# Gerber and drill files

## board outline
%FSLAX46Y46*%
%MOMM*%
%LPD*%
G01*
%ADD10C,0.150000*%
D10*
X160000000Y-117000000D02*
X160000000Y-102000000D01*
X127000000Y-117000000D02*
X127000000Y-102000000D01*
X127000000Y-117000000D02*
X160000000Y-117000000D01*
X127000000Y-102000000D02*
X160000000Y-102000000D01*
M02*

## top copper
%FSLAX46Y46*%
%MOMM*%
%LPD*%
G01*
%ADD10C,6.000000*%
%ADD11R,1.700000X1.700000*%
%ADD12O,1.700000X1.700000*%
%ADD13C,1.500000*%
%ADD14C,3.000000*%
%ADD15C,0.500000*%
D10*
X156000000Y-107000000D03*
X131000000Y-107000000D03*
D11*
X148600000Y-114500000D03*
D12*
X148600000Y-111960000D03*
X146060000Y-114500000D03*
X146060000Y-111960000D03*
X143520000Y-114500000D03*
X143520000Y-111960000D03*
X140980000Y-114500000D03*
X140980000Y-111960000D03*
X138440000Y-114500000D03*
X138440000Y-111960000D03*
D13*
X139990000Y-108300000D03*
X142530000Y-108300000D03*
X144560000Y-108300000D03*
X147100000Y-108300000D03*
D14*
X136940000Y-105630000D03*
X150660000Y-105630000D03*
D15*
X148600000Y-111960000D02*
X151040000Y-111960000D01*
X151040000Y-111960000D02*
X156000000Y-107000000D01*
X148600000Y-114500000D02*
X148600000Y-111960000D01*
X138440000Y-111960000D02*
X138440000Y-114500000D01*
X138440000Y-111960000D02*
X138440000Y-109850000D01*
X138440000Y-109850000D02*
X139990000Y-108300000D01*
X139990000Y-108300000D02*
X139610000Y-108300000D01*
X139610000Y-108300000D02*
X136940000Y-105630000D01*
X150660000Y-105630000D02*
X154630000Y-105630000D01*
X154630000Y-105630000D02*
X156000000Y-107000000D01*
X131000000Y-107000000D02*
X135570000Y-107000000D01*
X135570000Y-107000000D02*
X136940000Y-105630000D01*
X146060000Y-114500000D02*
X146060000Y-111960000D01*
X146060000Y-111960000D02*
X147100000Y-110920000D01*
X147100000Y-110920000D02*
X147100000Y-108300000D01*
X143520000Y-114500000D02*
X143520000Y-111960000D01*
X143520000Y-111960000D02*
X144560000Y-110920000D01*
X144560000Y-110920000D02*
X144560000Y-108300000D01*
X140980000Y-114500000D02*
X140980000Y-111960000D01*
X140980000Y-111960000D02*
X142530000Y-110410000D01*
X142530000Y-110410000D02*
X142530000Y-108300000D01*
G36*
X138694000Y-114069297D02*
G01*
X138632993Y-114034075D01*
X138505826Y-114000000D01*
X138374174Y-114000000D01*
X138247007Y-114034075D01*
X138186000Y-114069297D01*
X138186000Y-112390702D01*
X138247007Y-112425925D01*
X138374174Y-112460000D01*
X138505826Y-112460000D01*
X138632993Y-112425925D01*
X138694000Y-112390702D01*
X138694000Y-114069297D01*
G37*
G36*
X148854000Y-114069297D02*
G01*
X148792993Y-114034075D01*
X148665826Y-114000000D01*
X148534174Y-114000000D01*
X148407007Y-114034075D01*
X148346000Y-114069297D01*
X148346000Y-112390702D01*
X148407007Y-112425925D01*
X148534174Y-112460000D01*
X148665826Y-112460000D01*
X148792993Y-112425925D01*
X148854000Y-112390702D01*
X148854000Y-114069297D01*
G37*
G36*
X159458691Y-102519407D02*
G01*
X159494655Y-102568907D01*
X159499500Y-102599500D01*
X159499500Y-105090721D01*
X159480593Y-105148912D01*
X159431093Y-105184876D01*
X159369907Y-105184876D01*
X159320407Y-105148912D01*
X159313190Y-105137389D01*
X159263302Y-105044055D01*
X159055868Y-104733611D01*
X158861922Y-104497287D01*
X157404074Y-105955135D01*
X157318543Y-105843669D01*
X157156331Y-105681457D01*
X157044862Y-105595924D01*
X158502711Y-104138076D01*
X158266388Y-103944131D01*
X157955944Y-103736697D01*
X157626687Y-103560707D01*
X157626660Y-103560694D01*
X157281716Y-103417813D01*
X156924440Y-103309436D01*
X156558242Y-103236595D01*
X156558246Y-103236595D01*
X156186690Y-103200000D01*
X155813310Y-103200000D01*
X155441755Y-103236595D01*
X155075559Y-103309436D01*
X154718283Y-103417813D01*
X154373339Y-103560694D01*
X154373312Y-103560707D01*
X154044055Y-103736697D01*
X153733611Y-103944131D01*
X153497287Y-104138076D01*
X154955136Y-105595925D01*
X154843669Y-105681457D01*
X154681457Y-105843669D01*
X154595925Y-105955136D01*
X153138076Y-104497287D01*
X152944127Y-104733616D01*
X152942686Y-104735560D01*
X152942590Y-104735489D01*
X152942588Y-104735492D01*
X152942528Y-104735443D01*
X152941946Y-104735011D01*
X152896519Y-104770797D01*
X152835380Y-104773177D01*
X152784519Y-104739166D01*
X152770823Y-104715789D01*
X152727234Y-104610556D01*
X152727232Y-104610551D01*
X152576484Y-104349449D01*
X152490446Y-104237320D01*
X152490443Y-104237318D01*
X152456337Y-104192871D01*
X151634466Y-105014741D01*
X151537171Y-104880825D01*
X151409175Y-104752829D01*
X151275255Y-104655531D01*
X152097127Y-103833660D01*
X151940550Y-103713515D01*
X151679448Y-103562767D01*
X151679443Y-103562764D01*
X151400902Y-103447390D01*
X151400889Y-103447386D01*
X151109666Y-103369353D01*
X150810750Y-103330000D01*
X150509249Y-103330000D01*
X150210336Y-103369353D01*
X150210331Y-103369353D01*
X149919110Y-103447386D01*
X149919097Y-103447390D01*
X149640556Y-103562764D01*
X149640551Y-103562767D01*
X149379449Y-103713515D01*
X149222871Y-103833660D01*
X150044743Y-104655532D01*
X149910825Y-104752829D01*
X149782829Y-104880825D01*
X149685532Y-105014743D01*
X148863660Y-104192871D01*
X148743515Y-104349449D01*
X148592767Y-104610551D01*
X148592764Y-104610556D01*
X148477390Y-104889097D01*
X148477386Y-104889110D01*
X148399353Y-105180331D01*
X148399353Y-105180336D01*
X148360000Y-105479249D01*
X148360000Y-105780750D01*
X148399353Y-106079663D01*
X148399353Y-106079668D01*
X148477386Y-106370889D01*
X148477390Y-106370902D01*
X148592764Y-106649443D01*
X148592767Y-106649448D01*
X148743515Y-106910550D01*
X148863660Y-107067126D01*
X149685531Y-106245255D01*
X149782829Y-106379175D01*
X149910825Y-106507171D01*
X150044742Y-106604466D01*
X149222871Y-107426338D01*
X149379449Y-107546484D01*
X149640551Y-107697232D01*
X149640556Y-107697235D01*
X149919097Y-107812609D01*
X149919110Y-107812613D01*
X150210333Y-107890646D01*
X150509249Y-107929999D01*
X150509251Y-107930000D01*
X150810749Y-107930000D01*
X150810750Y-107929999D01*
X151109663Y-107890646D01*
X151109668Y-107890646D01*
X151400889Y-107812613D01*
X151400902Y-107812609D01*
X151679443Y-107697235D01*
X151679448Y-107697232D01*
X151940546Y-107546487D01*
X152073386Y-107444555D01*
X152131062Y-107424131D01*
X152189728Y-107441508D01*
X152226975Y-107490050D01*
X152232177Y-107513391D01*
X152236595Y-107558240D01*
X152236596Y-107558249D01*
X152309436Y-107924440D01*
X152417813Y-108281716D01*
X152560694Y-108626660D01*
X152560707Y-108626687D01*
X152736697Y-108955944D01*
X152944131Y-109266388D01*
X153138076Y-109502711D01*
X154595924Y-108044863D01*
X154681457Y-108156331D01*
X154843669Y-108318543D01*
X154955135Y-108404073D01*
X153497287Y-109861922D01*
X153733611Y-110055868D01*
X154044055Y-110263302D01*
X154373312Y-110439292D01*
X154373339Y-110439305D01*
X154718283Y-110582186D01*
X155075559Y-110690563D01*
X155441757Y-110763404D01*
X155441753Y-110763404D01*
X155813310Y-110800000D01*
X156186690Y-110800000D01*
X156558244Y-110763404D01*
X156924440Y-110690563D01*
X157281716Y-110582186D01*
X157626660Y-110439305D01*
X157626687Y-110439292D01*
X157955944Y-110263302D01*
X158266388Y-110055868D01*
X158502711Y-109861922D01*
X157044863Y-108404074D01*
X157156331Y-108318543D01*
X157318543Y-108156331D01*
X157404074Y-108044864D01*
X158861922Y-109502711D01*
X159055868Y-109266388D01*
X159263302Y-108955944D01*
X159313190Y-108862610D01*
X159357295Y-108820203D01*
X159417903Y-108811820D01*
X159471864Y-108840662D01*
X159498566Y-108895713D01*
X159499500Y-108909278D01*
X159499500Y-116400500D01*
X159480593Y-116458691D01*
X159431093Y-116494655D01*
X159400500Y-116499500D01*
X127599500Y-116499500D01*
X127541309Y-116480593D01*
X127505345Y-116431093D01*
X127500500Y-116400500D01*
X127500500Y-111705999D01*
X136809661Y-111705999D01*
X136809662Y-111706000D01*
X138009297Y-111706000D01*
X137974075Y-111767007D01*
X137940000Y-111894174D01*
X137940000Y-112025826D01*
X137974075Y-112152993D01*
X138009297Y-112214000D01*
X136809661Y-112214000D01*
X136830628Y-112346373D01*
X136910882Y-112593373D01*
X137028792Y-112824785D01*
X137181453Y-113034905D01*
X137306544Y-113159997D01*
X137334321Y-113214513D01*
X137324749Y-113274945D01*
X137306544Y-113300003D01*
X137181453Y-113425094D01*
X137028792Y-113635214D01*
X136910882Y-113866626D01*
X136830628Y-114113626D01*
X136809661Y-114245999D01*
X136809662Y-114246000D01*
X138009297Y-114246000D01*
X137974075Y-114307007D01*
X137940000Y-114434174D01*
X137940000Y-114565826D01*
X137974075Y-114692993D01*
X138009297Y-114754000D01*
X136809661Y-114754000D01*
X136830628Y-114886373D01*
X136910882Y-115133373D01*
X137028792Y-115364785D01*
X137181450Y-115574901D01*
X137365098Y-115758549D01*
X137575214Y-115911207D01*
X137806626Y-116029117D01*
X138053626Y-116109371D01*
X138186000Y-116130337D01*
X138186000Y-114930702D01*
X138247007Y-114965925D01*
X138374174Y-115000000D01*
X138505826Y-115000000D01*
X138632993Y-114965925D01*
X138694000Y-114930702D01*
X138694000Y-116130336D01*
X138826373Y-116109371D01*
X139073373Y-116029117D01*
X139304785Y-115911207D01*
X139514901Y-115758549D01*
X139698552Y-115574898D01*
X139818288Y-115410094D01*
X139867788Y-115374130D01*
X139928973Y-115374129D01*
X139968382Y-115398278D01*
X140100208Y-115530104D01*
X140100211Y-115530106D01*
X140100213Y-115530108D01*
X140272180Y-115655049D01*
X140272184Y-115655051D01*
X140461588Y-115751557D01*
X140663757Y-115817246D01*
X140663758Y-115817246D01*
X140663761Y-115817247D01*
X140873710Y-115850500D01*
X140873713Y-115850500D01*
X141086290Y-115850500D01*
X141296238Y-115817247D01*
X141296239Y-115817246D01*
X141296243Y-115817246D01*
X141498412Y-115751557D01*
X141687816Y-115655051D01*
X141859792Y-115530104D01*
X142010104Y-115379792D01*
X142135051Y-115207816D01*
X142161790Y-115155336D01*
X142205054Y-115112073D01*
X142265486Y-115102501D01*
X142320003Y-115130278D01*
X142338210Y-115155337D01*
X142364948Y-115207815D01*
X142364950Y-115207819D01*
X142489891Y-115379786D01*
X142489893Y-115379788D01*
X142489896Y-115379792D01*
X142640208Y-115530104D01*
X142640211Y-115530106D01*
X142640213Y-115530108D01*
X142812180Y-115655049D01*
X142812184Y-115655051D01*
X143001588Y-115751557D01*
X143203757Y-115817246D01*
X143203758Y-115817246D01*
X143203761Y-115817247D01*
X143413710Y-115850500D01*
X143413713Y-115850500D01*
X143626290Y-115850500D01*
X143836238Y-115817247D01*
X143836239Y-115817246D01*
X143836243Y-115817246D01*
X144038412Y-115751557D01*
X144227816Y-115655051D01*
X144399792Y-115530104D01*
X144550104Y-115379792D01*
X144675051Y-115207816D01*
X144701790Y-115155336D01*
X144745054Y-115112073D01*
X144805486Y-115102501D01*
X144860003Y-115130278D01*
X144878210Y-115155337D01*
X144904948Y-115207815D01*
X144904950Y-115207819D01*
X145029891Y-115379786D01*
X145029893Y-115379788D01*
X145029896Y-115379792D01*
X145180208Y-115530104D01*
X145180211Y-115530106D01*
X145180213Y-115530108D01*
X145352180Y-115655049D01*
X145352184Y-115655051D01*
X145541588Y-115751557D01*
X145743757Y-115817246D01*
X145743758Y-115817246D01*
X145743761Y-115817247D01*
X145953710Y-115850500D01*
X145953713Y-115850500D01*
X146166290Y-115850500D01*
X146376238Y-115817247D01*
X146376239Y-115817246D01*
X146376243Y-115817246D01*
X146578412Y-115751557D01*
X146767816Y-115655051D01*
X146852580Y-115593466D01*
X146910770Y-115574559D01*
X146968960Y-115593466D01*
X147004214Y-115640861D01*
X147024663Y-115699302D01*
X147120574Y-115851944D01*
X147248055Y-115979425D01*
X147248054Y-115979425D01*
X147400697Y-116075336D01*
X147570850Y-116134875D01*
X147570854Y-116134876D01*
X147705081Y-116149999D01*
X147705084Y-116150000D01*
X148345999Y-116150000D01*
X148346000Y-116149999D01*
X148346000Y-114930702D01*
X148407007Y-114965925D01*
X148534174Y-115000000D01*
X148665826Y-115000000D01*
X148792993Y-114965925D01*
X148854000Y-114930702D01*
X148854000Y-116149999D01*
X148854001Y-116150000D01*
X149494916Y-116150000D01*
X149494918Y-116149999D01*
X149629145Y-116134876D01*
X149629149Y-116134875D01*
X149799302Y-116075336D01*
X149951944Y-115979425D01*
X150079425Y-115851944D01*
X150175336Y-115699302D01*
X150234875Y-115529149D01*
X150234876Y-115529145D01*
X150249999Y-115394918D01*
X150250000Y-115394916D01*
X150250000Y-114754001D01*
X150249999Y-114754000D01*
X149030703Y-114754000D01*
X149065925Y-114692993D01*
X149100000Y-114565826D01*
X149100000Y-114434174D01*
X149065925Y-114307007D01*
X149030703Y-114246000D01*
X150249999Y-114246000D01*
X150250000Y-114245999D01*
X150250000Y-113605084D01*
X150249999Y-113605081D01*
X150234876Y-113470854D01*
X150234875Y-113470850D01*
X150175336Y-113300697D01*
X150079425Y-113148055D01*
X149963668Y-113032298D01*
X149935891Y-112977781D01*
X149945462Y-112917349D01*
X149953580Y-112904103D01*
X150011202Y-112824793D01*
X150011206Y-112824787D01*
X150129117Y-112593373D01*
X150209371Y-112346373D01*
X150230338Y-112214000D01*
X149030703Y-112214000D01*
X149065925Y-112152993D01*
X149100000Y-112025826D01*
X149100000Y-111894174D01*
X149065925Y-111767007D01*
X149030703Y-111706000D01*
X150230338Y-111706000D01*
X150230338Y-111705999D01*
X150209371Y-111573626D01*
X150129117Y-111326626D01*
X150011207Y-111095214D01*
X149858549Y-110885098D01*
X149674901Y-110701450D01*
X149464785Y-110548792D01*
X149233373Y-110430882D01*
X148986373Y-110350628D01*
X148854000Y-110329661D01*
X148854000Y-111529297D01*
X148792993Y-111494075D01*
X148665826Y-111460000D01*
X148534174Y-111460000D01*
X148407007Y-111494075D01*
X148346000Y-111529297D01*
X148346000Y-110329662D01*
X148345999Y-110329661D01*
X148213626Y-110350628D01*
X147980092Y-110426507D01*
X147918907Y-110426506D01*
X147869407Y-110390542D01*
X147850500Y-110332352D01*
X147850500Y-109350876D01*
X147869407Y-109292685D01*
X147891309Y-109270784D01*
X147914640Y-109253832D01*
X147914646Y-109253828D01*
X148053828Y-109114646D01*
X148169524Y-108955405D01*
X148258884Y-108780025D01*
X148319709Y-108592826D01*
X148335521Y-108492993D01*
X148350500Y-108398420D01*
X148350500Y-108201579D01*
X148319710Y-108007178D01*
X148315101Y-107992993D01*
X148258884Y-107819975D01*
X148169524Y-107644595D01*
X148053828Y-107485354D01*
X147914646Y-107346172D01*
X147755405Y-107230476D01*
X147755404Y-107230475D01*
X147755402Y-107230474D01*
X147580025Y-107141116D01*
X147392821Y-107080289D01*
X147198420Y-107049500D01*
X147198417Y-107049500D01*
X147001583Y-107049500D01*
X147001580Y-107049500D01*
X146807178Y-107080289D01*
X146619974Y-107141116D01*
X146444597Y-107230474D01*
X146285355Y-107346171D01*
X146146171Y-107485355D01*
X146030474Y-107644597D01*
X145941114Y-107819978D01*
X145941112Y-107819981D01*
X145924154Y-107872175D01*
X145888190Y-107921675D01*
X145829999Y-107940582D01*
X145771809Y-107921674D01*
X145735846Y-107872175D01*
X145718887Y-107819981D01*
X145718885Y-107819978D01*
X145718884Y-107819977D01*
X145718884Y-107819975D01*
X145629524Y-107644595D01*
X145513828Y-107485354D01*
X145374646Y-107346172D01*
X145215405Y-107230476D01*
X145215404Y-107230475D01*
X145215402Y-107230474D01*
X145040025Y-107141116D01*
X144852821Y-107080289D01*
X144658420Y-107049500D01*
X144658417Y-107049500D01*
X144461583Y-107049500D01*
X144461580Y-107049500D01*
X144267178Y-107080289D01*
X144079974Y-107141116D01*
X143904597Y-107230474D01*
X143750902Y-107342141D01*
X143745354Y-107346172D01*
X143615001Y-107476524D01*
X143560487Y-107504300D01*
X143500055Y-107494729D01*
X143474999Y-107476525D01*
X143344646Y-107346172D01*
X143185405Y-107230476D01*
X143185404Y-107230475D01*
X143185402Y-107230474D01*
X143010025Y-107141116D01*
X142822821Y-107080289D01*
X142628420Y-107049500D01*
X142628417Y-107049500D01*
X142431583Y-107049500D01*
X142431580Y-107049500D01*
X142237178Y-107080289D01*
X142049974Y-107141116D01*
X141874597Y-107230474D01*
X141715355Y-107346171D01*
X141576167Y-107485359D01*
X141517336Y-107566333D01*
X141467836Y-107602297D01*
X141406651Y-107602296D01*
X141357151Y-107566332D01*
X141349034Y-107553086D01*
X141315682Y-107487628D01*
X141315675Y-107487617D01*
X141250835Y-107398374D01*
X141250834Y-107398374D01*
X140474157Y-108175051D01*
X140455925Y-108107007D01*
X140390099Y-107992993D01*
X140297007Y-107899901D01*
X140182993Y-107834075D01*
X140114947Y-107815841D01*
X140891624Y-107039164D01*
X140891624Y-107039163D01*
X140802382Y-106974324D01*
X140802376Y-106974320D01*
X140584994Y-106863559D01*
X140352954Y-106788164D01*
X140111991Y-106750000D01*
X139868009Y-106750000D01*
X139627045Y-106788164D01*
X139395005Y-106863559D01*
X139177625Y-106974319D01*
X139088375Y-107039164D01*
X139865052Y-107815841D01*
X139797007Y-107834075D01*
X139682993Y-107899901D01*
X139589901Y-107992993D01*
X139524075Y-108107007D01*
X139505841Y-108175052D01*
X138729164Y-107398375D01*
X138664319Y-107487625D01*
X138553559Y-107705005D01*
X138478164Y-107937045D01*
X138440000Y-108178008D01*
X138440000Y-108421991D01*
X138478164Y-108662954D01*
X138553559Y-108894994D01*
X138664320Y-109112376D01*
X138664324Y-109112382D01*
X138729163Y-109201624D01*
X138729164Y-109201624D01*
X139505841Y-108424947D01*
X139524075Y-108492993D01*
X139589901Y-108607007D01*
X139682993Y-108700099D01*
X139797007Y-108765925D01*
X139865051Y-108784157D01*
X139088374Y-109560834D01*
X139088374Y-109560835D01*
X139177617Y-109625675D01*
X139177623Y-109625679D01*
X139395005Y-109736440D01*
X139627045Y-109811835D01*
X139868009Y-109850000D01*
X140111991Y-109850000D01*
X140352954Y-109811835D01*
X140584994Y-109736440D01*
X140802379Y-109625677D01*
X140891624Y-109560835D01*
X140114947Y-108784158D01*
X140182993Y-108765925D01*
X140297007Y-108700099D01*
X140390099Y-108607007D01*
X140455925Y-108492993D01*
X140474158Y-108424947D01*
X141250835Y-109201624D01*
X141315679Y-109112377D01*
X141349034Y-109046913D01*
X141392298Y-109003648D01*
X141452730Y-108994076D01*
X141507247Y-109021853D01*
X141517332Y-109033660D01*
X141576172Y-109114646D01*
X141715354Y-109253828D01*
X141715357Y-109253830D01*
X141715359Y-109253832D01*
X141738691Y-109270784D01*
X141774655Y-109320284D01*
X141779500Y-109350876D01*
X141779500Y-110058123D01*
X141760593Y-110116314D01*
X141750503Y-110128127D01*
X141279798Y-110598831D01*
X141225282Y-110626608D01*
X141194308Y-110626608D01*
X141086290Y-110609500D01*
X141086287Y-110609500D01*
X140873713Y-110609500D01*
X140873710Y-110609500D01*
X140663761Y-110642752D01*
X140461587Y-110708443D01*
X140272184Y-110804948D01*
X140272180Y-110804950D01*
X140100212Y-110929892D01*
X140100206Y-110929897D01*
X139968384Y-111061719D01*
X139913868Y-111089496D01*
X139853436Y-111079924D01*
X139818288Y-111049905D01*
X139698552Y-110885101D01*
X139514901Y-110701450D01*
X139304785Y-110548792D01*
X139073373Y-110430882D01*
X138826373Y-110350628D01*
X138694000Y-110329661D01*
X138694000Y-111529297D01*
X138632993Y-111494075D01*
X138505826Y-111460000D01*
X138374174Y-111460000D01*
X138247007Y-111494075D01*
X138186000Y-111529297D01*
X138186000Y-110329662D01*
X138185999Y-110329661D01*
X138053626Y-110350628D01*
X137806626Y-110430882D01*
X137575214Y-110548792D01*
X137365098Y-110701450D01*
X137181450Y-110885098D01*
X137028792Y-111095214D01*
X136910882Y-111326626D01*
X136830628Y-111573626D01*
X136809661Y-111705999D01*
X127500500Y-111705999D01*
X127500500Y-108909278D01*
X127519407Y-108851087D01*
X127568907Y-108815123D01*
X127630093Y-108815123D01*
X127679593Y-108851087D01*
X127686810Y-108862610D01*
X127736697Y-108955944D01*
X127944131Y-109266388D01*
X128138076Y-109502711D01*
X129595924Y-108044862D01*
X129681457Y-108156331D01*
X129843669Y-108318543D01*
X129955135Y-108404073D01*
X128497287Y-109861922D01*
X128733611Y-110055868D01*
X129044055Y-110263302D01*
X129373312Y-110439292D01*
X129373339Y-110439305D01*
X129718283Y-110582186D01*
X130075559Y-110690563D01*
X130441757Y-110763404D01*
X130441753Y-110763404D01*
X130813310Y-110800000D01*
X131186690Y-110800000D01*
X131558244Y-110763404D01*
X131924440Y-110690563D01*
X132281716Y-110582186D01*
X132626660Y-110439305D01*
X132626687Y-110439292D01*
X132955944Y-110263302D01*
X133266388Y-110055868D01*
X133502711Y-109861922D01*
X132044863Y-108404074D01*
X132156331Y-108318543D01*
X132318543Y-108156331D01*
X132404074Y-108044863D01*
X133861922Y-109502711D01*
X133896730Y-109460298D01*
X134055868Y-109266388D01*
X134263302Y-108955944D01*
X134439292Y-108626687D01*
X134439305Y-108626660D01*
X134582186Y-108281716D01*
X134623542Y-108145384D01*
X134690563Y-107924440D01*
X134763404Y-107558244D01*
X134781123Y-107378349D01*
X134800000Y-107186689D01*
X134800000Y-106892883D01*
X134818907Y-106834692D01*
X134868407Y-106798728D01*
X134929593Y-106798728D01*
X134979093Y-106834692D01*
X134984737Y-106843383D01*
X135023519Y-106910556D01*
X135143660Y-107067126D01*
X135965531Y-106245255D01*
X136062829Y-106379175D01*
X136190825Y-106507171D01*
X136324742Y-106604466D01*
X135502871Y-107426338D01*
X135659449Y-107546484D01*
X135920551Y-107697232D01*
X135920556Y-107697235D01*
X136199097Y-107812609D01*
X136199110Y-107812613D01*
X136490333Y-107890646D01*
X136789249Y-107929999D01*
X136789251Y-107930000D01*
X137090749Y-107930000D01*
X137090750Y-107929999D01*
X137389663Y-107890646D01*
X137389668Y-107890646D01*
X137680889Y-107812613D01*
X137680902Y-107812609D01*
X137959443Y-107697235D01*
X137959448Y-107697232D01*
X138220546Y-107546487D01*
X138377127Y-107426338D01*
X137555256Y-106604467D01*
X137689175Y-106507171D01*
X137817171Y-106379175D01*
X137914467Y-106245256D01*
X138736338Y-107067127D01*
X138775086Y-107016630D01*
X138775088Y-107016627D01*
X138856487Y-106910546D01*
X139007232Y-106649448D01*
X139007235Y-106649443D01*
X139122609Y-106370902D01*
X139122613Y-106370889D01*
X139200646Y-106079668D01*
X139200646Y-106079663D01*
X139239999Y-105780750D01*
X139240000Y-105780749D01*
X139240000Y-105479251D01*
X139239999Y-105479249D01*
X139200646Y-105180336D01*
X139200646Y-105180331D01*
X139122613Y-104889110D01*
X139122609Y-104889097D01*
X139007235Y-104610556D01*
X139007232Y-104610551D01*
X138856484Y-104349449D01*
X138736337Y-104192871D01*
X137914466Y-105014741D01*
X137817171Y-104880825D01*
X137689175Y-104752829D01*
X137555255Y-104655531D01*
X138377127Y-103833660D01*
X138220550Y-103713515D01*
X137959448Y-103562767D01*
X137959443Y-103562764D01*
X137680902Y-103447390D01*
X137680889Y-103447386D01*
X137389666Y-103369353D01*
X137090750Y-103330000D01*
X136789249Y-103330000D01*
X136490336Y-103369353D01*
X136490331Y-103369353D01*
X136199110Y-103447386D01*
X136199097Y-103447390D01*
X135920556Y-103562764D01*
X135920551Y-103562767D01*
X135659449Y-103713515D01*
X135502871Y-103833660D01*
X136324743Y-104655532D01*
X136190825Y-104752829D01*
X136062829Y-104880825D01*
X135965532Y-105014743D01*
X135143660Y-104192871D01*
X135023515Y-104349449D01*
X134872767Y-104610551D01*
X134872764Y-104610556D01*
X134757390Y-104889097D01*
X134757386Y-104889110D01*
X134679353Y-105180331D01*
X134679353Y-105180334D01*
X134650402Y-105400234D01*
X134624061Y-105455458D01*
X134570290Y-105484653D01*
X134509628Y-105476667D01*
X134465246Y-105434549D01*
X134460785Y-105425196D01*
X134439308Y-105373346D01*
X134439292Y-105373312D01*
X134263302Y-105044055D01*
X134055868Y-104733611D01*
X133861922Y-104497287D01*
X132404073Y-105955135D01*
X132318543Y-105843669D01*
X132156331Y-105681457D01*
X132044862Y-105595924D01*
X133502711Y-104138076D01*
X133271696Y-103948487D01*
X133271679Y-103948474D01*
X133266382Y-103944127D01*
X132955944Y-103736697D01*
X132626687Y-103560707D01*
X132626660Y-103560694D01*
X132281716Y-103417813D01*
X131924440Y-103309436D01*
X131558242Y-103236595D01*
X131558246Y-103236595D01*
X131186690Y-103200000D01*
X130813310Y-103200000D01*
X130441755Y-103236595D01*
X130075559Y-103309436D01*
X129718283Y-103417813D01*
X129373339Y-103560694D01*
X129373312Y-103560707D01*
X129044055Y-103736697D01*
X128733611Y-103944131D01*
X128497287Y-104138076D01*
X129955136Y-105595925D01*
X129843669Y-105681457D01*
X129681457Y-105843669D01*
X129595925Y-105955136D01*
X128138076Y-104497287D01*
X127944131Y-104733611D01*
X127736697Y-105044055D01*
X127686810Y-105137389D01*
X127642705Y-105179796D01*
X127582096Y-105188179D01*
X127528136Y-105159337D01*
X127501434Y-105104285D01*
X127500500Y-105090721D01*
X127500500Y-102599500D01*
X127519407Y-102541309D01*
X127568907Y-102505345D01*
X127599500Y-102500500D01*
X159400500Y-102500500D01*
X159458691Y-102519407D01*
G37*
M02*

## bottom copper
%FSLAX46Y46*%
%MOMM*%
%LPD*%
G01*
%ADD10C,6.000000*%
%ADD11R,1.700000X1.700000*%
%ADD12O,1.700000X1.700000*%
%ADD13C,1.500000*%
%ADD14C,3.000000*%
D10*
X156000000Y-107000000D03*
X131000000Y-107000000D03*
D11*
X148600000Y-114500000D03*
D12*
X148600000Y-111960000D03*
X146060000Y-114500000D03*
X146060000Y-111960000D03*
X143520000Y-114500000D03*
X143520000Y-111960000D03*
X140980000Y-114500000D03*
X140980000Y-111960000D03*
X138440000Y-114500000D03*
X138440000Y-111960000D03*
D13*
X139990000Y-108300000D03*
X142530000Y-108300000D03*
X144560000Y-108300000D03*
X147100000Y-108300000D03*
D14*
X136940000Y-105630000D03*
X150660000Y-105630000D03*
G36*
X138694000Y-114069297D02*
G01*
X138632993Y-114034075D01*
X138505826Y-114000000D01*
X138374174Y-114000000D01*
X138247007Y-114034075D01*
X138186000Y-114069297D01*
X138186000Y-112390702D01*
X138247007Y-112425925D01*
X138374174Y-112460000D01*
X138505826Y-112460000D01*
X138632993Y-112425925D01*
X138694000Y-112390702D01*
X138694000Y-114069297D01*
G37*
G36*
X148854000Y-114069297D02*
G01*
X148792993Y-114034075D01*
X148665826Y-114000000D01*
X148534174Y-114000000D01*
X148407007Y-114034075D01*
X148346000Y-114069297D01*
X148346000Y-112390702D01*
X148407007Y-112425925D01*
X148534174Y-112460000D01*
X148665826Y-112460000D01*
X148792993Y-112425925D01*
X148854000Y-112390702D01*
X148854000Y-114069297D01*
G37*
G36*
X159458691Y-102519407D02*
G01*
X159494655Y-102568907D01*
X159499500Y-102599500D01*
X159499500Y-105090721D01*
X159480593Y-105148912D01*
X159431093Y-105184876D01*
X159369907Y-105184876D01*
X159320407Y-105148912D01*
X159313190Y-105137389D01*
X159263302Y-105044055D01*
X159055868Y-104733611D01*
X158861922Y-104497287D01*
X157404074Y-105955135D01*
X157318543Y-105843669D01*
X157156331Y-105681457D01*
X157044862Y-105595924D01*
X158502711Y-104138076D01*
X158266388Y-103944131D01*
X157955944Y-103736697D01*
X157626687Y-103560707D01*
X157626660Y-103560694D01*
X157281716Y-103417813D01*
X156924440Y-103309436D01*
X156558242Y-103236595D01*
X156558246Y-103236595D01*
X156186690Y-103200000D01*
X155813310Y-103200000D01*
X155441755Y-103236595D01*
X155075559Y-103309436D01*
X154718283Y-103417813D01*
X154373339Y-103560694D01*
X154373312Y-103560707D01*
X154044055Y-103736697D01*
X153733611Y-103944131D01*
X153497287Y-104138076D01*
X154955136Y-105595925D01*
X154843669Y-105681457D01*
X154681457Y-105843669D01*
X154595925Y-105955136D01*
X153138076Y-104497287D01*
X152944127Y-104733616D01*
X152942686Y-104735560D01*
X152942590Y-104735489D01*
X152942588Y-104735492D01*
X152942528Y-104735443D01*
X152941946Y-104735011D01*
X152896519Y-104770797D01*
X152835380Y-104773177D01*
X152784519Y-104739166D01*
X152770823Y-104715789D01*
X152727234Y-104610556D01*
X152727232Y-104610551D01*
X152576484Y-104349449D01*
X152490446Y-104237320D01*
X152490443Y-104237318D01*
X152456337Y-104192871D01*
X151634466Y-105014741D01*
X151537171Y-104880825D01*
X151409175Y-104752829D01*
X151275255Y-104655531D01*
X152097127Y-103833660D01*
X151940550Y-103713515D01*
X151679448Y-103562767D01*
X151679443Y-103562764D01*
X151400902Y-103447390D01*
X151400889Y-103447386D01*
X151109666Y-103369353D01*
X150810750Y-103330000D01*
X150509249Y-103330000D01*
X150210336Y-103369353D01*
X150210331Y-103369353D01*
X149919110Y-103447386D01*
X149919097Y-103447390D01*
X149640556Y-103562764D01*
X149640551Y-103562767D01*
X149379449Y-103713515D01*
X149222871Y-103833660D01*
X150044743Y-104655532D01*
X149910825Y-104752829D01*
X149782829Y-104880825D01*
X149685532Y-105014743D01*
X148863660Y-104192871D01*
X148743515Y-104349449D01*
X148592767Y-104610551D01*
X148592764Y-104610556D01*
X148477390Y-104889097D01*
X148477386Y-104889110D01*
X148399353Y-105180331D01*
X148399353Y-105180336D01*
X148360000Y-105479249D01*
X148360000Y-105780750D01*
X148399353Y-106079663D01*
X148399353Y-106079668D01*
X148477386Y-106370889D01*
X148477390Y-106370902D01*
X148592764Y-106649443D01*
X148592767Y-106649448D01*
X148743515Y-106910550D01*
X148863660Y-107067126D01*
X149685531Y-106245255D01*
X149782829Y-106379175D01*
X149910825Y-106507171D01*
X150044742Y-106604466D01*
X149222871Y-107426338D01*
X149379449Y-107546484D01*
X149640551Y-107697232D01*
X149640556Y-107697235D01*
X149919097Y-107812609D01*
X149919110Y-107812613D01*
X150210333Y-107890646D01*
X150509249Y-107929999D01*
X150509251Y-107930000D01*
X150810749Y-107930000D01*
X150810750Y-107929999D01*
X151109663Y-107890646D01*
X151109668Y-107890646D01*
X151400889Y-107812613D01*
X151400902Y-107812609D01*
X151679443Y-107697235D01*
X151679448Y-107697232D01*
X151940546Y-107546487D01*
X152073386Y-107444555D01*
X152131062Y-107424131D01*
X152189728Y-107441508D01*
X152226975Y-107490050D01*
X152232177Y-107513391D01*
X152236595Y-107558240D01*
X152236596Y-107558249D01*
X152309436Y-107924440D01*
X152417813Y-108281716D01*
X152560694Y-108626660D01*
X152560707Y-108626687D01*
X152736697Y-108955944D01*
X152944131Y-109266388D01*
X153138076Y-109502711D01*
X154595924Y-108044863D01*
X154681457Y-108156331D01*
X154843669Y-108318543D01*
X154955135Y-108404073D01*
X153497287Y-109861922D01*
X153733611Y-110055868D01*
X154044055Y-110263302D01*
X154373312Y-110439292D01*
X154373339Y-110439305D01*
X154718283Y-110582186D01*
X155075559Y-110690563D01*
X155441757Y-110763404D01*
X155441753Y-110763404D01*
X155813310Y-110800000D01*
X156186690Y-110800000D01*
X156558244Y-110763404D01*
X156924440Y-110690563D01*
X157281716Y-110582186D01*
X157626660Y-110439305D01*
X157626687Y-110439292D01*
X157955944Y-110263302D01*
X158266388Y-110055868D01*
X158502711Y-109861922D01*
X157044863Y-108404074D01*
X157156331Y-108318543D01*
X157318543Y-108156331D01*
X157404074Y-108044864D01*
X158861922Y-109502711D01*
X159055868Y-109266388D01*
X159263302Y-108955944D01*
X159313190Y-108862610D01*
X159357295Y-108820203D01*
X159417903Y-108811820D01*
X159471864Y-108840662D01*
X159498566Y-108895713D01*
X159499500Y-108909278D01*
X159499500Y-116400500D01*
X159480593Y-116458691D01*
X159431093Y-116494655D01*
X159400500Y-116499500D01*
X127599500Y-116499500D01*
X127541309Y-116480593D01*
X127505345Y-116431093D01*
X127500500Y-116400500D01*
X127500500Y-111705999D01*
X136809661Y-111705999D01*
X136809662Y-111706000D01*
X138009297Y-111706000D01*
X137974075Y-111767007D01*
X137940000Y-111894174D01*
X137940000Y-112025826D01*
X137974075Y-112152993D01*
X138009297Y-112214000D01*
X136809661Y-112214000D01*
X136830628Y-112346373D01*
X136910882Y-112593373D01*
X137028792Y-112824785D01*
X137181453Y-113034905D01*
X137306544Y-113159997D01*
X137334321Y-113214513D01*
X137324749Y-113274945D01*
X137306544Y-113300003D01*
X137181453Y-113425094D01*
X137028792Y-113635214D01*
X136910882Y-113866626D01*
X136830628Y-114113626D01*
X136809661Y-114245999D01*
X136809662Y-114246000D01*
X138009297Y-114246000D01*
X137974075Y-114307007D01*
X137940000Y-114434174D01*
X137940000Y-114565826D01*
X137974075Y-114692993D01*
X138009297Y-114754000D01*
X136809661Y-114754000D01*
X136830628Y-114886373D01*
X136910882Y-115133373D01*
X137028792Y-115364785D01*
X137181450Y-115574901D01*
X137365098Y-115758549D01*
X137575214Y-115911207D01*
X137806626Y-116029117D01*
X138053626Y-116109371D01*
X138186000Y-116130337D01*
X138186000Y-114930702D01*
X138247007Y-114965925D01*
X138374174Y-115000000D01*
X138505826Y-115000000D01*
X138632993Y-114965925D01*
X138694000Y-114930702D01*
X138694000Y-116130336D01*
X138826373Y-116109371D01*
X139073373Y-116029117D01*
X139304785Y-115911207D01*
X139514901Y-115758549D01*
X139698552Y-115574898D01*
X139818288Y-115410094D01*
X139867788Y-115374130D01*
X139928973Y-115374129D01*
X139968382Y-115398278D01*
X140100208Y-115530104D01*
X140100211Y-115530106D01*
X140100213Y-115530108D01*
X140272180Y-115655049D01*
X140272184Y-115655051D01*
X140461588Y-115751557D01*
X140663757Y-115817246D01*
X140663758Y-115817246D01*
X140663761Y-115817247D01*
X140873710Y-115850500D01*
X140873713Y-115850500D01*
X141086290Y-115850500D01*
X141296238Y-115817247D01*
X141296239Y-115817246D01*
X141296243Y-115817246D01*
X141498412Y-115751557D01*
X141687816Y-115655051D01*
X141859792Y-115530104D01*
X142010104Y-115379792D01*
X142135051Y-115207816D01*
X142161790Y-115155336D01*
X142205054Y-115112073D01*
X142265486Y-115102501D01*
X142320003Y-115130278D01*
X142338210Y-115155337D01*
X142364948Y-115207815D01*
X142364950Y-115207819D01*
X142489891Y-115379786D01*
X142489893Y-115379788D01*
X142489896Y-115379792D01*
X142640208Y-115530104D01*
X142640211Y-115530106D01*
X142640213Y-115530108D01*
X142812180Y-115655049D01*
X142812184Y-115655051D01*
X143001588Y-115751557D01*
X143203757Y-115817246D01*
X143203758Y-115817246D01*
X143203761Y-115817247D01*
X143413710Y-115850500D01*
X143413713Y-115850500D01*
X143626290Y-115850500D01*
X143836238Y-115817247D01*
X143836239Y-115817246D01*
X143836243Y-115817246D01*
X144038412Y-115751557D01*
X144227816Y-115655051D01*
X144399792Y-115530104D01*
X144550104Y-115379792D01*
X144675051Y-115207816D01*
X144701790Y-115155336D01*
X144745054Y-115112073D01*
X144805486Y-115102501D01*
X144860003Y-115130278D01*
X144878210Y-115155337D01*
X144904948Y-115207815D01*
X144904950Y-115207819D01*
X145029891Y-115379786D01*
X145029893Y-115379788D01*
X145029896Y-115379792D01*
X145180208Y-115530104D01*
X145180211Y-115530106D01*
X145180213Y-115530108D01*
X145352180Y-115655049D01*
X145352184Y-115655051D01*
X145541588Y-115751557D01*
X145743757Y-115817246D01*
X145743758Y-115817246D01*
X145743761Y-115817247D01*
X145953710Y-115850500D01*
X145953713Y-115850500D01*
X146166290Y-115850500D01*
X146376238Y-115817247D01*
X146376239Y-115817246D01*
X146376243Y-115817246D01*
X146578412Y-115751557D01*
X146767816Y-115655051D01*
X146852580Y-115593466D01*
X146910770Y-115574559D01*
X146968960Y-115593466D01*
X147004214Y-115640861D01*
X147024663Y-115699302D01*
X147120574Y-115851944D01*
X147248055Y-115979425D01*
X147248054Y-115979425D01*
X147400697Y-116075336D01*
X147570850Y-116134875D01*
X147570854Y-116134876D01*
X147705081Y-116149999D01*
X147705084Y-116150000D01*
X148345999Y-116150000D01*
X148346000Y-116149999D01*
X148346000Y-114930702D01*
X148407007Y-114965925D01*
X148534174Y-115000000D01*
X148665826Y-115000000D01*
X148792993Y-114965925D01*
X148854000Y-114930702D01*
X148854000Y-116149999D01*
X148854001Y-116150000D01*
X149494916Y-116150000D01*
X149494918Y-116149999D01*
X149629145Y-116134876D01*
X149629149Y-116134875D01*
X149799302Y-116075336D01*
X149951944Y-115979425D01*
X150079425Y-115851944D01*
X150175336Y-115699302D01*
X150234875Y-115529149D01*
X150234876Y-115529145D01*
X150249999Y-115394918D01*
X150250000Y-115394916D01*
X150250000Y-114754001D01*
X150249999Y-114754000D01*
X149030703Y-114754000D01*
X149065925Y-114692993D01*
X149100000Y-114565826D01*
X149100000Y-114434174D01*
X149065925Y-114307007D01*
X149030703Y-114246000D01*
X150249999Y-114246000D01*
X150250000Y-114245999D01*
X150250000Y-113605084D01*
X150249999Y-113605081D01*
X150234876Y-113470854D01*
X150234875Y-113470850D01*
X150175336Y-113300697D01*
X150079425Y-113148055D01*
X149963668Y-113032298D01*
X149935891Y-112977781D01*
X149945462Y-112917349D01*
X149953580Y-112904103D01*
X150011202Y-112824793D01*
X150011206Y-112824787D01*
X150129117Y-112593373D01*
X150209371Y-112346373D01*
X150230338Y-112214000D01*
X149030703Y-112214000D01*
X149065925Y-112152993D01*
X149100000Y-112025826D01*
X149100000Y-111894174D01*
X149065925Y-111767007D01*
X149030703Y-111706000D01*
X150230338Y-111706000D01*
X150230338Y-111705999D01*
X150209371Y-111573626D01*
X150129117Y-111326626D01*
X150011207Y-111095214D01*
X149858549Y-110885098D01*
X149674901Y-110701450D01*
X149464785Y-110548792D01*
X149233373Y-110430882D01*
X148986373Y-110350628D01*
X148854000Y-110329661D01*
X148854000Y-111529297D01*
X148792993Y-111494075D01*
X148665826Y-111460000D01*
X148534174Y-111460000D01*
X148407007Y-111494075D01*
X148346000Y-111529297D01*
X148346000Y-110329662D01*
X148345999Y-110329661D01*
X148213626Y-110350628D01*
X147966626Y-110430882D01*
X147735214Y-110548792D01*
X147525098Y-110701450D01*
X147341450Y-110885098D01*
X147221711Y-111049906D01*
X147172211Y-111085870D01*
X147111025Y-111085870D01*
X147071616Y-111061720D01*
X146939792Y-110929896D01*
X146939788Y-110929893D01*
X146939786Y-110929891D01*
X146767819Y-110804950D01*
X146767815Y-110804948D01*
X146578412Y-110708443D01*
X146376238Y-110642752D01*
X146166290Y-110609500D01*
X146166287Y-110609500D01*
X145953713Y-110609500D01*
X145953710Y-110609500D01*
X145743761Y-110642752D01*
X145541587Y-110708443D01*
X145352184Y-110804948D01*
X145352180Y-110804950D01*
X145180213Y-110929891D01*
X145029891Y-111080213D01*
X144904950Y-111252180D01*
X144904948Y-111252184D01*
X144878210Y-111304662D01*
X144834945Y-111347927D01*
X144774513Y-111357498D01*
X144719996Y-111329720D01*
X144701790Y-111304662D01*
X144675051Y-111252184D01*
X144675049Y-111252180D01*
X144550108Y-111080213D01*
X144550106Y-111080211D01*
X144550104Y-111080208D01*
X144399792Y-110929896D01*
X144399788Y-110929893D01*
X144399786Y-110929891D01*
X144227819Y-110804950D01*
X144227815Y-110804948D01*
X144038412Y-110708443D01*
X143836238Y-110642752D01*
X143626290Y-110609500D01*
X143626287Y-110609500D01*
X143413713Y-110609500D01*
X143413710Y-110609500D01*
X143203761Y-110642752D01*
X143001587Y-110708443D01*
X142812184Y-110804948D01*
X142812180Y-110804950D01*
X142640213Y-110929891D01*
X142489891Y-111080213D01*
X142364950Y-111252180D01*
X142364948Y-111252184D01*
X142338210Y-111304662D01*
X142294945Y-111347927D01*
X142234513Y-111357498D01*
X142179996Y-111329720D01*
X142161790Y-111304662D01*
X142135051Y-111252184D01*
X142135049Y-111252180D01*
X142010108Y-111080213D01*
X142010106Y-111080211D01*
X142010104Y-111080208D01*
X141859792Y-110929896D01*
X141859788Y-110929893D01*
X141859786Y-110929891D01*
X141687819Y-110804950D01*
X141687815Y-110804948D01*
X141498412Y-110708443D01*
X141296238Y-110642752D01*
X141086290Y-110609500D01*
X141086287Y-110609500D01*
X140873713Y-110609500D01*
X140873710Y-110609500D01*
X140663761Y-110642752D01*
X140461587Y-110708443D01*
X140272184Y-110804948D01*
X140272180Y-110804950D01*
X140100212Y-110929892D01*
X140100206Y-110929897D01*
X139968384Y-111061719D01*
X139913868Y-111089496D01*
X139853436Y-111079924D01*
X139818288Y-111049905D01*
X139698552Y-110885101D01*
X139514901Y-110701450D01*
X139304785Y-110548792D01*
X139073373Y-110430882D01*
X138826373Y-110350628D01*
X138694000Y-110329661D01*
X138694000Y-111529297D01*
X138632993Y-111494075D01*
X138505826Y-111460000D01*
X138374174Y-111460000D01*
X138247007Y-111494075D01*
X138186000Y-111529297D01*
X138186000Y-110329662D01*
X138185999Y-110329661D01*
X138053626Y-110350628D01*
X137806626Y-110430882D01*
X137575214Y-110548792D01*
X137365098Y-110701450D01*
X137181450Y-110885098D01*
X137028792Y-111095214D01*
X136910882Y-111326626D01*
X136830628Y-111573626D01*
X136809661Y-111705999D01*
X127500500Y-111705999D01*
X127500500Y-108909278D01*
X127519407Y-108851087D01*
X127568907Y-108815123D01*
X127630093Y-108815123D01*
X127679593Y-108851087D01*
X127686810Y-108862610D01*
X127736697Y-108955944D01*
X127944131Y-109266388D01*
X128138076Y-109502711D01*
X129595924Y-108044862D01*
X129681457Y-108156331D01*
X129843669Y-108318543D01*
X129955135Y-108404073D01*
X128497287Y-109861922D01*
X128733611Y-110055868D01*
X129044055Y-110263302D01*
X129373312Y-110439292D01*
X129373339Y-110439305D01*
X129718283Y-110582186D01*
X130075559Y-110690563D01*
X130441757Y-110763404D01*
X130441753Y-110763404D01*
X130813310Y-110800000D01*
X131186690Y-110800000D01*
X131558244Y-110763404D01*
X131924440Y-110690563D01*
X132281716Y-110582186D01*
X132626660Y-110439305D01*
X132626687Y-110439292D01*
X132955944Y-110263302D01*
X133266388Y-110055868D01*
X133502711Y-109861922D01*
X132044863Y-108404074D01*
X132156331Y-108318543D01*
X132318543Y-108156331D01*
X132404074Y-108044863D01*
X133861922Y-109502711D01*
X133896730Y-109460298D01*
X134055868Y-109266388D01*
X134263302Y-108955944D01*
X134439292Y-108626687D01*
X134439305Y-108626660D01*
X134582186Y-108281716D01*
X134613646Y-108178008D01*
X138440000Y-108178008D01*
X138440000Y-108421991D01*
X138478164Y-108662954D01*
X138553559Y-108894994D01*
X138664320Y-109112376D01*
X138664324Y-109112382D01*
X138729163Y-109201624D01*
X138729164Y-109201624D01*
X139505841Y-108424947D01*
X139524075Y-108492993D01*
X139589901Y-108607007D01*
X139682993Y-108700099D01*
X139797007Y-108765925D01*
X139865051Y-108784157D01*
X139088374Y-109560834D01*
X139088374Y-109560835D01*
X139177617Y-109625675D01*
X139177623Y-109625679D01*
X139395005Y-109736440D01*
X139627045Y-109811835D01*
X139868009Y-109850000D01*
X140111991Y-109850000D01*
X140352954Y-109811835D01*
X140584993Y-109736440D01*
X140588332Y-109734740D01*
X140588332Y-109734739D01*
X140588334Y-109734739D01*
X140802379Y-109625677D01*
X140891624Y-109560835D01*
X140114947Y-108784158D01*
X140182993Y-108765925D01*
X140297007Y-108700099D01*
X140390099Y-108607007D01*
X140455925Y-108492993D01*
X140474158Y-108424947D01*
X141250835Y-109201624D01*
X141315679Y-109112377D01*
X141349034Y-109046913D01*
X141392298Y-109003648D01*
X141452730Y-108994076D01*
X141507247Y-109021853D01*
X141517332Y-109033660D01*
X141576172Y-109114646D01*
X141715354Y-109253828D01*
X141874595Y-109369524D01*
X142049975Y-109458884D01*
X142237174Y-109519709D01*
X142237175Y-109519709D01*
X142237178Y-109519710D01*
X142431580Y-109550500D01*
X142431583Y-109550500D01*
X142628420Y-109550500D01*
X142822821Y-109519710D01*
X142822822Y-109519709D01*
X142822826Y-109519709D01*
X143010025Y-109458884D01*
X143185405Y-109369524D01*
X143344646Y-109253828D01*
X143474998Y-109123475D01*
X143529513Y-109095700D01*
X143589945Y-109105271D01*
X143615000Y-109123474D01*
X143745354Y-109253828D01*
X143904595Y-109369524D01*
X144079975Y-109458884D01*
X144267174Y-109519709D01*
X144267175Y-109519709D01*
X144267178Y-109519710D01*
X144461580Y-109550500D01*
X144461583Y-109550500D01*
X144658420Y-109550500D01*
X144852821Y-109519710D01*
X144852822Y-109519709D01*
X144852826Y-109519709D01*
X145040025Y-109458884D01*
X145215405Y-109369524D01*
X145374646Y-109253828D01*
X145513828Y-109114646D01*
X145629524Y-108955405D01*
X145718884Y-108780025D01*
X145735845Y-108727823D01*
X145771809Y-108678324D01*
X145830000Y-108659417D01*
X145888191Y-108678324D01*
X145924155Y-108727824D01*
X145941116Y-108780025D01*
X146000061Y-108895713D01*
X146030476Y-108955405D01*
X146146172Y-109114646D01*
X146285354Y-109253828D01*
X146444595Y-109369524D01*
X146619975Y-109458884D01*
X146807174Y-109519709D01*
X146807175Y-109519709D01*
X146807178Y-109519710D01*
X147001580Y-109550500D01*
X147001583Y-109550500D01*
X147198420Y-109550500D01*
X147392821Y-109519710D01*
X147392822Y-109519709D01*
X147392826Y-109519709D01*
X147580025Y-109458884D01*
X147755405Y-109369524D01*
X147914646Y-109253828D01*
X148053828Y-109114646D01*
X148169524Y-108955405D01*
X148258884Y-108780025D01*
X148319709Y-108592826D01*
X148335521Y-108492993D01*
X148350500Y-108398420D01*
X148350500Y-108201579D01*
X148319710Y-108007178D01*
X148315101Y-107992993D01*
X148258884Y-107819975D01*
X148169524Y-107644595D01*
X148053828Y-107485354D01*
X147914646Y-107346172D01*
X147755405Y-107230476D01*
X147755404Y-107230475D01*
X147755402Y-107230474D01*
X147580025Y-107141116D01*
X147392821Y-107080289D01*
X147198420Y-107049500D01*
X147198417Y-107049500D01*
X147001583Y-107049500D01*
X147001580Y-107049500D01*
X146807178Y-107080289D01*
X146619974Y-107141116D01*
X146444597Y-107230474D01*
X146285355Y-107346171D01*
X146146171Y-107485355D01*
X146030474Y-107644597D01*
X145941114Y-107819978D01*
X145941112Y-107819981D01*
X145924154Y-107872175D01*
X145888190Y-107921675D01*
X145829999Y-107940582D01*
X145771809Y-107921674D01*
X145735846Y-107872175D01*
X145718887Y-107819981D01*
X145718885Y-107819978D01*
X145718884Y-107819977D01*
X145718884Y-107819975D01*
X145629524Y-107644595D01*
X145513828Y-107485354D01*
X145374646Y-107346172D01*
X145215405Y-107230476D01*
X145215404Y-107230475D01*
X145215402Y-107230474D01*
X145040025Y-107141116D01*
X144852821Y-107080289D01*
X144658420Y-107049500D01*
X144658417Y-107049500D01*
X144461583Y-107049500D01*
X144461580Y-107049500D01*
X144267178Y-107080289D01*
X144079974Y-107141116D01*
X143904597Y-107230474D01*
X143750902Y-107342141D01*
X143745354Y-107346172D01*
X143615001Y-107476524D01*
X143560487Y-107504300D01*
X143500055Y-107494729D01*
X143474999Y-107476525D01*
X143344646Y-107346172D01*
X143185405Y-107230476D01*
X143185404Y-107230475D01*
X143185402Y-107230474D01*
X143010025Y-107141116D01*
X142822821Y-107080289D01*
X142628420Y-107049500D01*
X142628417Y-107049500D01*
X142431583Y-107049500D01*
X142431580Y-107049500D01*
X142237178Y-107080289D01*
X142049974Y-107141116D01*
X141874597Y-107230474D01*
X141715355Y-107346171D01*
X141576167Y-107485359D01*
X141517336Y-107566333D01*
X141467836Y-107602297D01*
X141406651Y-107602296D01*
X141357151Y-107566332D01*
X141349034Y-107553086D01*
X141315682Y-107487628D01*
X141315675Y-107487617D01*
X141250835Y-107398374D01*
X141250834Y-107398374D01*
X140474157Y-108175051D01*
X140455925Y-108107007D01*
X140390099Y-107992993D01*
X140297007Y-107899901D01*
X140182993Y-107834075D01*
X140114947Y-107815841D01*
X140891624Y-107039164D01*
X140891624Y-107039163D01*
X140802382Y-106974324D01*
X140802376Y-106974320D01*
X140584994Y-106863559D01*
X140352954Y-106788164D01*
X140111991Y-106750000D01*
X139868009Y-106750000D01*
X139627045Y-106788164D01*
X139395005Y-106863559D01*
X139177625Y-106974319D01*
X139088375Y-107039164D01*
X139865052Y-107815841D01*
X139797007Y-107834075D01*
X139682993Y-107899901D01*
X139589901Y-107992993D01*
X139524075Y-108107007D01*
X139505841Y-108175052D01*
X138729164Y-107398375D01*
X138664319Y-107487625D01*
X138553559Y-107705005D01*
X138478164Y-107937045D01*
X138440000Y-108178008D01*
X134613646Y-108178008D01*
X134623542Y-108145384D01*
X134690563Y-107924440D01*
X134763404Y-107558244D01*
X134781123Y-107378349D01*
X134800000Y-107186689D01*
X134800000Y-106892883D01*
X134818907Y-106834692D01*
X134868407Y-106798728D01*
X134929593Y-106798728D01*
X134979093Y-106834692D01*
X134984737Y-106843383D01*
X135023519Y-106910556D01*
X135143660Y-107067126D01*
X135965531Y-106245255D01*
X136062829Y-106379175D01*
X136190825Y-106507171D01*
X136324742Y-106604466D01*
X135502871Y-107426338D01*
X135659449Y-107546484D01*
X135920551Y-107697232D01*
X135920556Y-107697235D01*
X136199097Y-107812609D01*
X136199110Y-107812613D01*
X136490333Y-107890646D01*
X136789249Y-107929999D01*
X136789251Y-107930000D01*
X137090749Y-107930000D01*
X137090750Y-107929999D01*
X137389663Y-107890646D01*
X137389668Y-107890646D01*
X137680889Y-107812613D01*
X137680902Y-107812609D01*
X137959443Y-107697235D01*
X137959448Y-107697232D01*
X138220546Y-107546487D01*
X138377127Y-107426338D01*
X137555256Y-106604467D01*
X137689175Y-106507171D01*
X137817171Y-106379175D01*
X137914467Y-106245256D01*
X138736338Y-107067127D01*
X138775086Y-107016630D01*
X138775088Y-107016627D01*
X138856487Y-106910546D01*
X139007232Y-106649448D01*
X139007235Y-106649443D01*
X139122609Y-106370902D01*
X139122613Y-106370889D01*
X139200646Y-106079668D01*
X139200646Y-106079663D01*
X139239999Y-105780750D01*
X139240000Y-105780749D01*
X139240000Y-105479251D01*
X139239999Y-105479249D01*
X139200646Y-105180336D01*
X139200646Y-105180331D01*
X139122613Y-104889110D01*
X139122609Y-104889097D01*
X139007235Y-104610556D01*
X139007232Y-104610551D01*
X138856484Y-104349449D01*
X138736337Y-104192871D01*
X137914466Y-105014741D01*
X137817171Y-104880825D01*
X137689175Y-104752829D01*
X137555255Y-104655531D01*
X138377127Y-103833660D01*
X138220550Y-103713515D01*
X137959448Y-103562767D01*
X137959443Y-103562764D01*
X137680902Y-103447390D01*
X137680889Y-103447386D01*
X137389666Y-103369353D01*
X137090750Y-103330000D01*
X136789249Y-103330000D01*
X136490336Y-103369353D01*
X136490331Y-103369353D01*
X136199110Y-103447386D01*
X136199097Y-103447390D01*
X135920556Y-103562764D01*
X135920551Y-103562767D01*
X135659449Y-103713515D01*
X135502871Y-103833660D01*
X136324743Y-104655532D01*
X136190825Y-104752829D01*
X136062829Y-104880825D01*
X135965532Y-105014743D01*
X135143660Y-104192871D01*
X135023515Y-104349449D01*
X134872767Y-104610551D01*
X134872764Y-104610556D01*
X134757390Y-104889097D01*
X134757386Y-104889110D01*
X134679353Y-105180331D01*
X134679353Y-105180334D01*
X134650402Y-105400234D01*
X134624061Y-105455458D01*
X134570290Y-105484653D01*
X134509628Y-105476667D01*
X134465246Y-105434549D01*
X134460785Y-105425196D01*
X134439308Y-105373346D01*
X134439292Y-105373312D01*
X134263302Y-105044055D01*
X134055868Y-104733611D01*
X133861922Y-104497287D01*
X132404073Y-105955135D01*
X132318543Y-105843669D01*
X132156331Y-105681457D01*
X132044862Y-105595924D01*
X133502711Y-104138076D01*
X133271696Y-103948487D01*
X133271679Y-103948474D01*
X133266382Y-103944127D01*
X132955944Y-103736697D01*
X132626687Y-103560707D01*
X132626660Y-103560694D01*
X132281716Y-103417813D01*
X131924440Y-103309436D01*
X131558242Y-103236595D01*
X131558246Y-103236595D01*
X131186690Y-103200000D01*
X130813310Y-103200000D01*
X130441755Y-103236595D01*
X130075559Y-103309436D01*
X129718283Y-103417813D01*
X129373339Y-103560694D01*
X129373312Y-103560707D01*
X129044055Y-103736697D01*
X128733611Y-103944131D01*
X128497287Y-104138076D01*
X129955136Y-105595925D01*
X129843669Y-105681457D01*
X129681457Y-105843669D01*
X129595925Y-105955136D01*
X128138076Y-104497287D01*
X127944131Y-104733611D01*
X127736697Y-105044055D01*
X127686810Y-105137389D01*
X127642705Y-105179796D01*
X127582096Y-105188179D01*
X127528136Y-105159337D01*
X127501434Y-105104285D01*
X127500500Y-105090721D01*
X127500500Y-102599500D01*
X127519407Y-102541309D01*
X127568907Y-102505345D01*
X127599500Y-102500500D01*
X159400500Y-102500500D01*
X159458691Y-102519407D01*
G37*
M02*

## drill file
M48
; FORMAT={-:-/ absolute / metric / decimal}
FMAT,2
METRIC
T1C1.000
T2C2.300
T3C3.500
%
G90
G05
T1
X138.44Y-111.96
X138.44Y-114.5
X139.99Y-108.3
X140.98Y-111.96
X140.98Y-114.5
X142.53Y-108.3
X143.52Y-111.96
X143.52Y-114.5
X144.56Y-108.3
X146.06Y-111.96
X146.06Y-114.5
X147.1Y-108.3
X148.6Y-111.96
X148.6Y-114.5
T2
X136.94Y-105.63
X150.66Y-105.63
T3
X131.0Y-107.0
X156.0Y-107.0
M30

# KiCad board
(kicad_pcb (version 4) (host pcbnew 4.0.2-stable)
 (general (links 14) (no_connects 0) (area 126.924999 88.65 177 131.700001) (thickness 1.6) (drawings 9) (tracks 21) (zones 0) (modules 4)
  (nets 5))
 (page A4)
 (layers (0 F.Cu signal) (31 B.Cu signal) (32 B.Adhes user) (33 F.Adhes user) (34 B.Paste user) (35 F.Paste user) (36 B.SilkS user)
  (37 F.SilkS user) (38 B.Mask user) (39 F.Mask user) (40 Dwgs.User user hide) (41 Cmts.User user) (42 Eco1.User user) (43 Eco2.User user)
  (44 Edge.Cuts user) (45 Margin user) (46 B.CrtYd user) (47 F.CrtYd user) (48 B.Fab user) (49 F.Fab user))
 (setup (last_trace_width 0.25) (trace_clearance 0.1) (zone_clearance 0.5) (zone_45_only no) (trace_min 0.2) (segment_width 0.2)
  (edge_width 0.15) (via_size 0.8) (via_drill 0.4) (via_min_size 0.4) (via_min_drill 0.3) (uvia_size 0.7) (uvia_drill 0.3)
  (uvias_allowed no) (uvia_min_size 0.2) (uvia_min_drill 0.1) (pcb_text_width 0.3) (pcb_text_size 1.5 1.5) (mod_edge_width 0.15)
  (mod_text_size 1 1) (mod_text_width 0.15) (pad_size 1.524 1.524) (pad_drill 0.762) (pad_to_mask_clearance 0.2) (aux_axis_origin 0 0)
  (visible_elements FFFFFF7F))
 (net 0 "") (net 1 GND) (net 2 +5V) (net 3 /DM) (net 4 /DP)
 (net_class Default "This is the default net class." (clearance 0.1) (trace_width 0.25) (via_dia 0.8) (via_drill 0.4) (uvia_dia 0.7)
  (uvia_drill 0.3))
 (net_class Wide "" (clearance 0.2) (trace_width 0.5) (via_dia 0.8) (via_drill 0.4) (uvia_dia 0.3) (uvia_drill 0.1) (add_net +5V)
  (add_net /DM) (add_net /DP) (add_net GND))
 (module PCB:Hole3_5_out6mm (layer F.Cu) (at 156 107)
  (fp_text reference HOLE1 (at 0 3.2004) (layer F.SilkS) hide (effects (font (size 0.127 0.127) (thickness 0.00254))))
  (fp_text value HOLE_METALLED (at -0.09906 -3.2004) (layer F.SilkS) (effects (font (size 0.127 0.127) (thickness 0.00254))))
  (pad H thru_hole circle (at 0 0) (size 6 6) (drill 3.5) (layers *.Cu *.Mask F.SilkS) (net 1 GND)))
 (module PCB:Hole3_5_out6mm (layer F.Cu) (at 131 107)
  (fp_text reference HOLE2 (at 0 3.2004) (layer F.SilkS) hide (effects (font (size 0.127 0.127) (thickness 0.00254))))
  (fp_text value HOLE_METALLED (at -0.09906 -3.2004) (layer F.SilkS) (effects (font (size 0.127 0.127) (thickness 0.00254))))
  (pad H thru_hole circle (at 0 0) (size 6 6) (drill 3.5) (layers *.Cu *.Mask F.SilkS) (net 1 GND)))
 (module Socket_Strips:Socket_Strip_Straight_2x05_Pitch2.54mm (layer F.Cu) (at 148.6 114.5 270)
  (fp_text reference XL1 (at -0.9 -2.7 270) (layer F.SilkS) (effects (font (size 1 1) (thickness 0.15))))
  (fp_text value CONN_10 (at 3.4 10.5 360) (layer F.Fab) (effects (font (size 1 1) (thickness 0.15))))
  (pad 1 thru_hole rect (at 0 0 270) (size 1.7 1.7) (drill 1) (layers *.Cu *.Mask) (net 1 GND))
  (pad 2 thru_hole oval (at -2.54 0 270) (size 1.7 1.7) (drill 1) (layers *.Cu *.Mask) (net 1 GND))
  (pad 3 thru_hole oval (at 0 2.54 270) (size 1.7 1.7) (drill 1) (layers *.Cu *.Mask) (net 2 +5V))
  (pad 4 thru_hole oval (at -2.54 2.54 270) (size 1.7 1.7) (drill 1) (layers *.Cu *.Mask) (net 2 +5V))
  (pad 5 thru_hole oval (at 0 5.08 270) (size 1.7 1.7) (drill 1) (layers *.Cu *.Mask) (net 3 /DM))
  (pad 6 thru_hole oval (at -2.54 5.08 270) (size 1.7 1.7) (drill 1) (layers *.Cu *.Mask) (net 3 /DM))
  (pad 7 thru_hole oval (at 0 7.62 270) (size 1.7 1.7) (drill 1) (layers *.Cu *.Mask) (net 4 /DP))
  (pad 8 thru_hole oval (at -2.54 7.62 270) (size 1.7 1.7) (drill 1) (layers *.Cu *.Mask) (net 4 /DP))
  (pad 9 thru_hole oval (at 0 10.16 270) (size 1.7 1.7) (drill 1) (layers *.Cu *.Mask) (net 1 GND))
  (pad 10 thru_hole oval (at -2.54 10.16 270) (size 1.7 1.7) (drill 1) (layers *.Cu *.Mask) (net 1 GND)))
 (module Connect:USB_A (layer F.Cu) (at 147.1 108.3 180)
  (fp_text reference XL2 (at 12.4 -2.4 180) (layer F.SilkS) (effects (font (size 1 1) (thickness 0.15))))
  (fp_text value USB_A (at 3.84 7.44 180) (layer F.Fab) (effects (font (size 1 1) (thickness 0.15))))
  (pad 4 thru_hole circle (at 7.11 0 90) (size 1.5 1.5) (drill 1) (layers *.Cu *.Mask) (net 1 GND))
  (pad 3 thru_hole circle (at 4.57 0 90) (size 1.5 1.5) (drill 1) (layers *.Cu *.Mask) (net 4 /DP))
  (pad 2 thru_hole circle (at 2.54 0 90) (size 1.5 1.5) (drill 1) (layers *.Cu *.Mask) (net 3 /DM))
  (pad 1 thru_hole circle (at 0 0 90) (size 1.5 1.5) (drill 1) (layers *.Cu *.Mask) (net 2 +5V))
  (pad 5 thru_hole circle (at 10.16 2.67 90) (size 3 3) (drill 2.3) (layers *.Cu *.Mask) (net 1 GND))
  (pad 5 thru_hole circle (at -3.56 2.67 90) (size 3 3) (drill 2.3) (layers *.Cu *.Mask) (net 1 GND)))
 (gr_line (start 160 117) (end 160 102) (angle 90) (layer Edge.Cuts) (width 0.15))
 (gr_line (start 127 117) (end 127 102) (angle 90) (layer Edge.Cuts) (width 0.15))
 (gr_line (start 127 117) (end 160 117) (angle 90) (layer Edge.Cuts) (width 0.15))
 (gr_line (start 127 102) (end 160 102) (angle 90) (layer Edge.Cuts) (width 0.15))
 (segment (start 148.6 111.96) (end 151.04 111.96) (width 0.5) (layer F.Cu) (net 1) (status 400000))
 (segment (start 151.04 111.96) (end 156 107) (width 0.5) (layer F.Cu) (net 1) (status 800000))
 (segment (start 148.6 114.5) (end 148.6 111.96) (width 0.5) (layer F.Cu) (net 1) (status C00000))
 (segment (start 138.44 111.96) (end 138.44 114.5) (width 0.5) (layer F.Cu) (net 1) (status C00000))
 (segment (start 138.44 111.96) (end 138.44 109.85) (width 0.5) (layer F.Cu) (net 1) (status 400000))
 (segment (start 138.44 109.85) (end 139.99 108.3) (width 0.5) (layer F.Cu) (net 1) (status 800000))
 (segment (start 139.99 108.3) (end 139.61 108.3) (width 0.5) (layer F.Cu) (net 1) (status C00000))
 (segment (start 139.61 108.3) (end 136.94 105.63) (width 0.5) (layer F.Cu) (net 1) (status C00000))
 (segment (start 150.66 105.63) (end 154.63 105.63) (width 0.5) (layer F.Cu) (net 1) (status C00000))
 (segment (start 154.63 105.63) (end 156 107) (width 0.5) (layer F.Cu) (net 1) (status C00000))
 (segment (start 131 107) (end 135.57 107) (width 0.5) (layer F.Cu) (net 1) (status 400000))
 (segment (start 135.57 107) (end 136.94 105.63) (width 0.5) (layer F.Cu) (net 1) (status 800000))
 (segment (start 146.06 114.5) (end 146.06 111.96) (width 0.5) (layer F.Cu) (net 2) (status C00000))
 (segment (start 146.06 111.96) (end 147.1 110.92) (width 0.5) (layer F.Cu) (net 2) (status 400000))
 (segment (start 147.1 110.92) (end 147.1 108.3) (width 0.5) (layer F.Cu) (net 2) (status 800000))
 (segment (start 143.52 114.5) (end 143.52 111.96) (width 0.5) (layer F.Cu) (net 3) (status C00000))
 (segment (start 143.52 111.96) (end 144.56 110.92) (width 0.5) (layer F.Cu) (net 3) (status 400000))
 (segment (start 144.56 110.92) (end 144.56 108.3) (width 0.5) (layer F.Cu) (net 3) (status 800000))
 (segment (start 140.98 114.5) (end 140.98 111.96) (width 0.5) (layer F.Cu) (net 4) (status C00000))
 (segment (start 140.98 111.96) (end 142.53 110.41) (width 0.5) (layer F.Cu) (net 4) (status 400000))
 (segment (start 142.53 110.41) (end 142.53 108.3) (width 0.5) (layer F.Cu) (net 4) (status 800000))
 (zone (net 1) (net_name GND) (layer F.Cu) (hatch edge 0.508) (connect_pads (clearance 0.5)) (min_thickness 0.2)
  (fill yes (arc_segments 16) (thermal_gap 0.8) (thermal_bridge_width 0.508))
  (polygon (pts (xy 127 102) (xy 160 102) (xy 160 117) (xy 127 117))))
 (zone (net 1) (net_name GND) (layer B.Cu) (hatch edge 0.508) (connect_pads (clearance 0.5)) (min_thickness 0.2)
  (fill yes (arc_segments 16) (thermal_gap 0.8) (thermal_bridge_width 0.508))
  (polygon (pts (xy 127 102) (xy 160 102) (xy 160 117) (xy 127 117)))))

